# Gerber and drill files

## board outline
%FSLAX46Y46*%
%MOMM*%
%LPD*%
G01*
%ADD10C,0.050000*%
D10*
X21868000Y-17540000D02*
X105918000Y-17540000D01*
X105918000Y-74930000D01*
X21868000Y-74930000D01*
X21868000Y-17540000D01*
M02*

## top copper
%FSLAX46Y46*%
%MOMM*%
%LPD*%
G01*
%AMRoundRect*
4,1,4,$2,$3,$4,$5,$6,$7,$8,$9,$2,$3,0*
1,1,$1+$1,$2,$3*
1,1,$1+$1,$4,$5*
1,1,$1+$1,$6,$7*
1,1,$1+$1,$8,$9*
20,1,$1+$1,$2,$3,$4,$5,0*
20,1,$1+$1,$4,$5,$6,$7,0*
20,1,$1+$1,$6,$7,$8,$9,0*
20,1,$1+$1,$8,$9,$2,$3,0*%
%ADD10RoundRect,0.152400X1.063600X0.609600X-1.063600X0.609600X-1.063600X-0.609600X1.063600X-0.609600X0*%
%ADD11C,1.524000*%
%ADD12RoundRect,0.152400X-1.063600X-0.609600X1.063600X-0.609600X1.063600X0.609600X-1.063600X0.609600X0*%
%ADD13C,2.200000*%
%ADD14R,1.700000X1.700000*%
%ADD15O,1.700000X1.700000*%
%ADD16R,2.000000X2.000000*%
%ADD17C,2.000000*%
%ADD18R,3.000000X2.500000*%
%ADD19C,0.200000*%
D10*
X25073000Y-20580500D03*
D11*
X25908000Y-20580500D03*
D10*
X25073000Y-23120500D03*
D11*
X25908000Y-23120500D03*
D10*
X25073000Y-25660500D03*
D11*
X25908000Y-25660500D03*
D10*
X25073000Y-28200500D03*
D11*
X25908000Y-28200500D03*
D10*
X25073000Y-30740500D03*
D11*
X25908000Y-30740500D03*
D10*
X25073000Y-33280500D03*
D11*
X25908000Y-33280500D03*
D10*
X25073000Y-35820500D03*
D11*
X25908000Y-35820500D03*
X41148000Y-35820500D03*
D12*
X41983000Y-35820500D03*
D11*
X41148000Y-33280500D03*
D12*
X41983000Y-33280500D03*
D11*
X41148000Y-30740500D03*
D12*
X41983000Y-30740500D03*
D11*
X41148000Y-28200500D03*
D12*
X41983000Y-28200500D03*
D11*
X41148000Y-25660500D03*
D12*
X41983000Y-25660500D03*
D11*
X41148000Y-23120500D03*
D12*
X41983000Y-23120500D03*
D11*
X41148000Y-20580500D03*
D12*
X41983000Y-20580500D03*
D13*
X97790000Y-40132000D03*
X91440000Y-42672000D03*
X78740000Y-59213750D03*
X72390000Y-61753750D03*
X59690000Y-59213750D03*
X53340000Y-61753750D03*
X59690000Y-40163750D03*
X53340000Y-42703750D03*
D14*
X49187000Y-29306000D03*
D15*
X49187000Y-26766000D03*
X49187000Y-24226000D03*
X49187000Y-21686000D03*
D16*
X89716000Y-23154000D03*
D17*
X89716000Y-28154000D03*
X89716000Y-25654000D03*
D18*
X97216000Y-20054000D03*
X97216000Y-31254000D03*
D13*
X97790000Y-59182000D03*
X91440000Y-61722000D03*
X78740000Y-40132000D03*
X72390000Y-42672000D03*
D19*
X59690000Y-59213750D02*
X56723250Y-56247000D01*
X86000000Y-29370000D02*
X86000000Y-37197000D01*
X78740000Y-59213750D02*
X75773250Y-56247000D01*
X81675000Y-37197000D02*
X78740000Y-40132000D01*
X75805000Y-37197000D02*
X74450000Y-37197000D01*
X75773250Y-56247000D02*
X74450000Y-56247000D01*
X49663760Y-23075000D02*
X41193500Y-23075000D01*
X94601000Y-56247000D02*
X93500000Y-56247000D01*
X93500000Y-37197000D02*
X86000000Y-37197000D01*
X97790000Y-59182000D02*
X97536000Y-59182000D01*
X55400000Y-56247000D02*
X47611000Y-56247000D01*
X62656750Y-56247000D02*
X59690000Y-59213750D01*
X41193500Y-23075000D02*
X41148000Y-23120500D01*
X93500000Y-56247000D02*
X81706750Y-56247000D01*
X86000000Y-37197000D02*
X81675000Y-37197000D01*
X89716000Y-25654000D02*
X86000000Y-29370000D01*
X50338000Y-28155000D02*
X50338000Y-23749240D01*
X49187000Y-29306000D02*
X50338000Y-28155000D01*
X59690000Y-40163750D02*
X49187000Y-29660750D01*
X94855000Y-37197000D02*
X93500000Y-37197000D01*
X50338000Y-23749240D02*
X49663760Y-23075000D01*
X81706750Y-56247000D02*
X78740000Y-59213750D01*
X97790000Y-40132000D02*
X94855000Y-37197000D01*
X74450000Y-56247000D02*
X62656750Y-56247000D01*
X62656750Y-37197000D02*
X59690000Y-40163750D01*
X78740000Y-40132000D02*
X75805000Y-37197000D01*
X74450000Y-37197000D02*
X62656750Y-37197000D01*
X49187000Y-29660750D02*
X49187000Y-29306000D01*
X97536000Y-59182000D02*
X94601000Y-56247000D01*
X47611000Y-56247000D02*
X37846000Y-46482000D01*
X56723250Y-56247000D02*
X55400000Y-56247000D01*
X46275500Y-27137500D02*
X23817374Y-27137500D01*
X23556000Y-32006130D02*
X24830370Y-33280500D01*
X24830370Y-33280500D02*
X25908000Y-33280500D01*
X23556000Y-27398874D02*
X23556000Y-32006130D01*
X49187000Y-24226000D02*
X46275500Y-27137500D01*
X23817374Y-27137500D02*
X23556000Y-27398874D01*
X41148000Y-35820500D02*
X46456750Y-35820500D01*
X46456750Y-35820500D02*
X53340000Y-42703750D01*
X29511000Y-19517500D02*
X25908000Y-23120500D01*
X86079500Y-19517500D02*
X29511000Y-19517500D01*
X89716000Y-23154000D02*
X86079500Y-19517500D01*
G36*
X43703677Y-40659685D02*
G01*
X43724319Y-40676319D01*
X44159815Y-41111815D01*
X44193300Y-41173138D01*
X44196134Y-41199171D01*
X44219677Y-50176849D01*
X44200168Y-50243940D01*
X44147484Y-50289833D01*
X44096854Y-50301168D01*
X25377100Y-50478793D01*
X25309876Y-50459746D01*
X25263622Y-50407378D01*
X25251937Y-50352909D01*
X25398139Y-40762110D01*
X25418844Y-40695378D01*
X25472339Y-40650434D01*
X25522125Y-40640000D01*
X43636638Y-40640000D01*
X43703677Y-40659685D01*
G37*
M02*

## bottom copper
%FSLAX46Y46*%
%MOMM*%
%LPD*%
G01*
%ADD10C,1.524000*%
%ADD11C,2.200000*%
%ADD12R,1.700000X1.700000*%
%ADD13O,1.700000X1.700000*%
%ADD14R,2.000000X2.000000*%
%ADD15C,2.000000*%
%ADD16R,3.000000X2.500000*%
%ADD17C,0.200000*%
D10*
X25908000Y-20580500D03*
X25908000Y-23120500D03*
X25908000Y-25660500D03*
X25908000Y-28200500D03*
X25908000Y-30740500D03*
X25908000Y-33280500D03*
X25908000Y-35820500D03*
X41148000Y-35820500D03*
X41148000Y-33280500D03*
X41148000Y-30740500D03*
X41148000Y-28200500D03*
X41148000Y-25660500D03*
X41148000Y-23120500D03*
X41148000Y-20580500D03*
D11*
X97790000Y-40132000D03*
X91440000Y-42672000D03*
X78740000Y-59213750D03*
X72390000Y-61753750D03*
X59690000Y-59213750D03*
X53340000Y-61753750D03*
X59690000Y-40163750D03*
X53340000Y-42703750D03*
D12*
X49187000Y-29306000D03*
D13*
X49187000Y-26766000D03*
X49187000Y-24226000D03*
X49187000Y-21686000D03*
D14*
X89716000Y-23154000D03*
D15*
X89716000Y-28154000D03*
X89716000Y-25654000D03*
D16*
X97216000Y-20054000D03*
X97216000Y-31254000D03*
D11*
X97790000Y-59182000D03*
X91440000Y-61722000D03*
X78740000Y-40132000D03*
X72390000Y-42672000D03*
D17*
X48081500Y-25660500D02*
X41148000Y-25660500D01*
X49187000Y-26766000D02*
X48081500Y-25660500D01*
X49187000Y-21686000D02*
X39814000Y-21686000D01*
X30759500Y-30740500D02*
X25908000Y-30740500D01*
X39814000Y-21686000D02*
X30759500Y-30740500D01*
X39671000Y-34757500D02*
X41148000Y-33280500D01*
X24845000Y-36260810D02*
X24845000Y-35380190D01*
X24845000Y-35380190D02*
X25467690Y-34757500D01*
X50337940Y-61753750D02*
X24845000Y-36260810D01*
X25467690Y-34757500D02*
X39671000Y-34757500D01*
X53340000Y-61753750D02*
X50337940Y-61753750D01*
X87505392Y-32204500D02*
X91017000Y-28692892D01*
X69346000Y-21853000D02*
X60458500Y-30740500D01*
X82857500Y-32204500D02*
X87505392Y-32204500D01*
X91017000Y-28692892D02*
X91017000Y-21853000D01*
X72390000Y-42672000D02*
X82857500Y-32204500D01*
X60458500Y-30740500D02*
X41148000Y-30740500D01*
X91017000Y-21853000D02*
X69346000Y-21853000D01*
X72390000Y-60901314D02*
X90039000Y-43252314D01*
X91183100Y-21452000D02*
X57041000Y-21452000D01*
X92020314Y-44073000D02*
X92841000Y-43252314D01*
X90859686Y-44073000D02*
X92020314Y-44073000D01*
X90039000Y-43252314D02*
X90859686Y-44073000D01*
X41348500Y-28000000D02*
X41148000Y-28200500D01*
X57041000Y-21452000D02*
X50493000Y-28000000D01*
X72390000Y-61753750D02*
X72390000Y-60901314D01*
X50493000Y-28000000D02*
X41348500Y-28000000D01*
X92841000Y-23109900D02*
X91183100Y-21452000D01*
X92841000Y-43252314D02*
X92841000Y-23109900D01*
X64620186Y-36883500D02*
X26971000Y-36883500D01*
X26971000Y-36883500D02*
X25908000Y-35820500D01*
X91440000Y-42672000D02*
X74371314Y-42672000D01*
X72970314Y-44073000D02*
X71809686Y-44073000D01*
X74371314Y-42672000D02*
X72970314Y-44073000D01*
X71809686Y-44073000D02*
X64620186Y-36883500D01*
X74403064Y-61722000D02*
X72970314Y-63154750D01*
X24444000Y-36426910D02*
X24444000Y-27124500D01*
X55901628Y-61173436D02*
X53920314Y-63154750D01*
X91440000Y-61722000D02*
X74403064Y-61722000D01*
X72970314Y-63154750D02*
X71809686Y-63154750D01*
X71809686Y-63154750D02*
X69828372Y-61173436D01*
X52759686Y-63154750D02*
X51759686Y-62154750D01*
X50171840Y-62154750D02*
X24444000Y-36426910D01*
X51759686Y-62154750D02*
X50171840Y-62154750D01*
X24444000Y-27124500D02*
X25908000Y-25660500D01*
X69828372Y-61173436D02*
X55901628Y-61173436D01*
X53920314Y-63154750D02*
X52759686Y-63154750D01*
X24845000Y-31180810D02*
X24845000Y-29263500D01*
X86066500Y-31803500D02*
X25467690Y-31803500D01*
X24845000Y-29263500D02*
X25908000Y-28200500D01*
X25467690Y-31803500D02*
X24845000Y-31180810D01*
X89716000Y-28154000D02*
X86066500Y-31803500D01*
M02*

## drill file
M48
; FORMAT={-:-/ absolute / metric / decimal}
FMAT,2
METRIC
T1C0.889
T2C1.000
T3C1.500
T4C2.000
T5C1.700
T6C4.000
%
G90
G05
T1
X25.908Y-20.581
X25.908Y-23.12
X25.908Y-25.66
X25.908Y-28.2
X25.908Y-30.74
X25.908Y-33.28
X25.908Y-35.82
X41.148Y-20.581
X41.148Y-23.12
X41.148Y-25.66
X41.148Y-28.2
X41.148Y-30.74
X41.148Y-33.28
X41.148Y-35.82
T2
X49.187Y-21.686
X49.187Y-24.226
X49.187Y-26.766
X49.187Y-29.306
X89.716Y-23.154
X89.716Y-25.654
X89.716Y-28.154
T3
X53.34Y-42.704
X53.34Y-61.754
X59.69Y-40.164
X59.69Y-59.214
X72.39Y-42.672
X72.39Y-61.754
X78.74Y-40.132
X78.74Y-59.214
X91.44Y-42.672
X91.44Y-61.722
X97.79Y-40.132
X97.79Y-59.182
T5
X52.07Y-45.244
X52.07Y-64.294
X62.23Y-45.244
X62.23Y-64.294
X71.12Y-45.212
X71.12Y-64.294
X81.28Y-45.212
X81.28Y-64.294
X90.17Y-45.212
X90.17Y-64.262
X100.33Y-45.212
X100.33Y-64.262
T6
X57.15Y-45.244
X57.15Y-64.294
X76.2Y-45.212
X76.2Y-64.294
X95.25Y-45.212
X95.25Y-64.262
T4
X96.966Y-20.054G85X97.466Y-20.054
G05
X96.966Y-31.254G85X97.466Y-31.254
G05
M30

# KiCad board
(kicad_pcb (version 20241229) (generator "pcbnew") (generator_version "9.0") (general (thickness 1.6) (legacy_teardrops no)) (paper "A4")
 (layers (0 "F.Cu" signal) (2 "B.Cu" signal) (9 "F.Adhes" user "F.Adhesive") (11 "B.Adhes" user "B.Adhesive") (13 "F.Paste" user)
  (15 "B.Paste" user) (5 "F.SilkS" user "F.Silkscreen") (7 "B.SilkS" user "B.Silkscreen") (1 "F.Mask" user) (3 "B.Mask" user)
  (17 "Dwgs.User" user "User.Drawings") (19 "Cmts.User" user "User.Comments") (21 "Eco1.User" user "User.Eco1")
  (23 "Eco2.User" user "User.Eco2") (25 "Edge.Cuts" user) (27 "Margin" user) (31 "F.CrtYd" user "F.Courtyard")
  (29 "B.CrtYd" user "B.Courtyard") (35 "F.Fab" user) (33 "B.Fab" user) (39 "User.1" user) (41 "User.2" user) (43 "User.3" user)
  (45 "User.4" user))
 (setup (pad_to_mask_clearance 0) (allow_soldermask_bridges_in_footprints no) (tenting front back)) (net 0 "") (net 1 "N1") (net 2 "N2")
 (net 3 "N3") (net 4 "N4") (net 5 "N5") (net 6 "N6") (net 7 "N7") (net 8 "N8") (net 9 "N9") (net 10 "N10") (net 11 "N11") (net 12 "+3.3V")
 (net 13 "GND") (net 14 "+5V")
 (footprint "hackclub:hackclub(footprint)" (layer "F.Cu") (at 35 58.15)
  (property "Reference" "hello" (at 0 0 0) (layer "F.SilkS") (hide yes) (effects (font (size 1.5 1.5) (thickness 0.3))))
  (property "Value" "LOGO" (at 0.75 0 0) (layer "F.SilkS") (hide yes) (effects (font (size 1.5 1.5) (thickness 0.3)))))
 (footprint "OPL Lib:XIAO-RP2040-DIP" (layer "F.Cu") (at 33.528 28.2005)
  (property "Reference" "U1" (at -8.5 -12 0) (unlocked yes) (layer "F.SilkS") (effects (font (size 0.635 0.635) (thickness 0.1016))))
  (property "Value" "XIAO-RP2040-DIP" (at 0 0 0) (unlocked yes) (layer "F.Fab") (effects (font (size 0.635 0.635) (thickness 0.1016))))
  (pad "1" smd roundrect (at -8.455 -7.62 180) (size 2.432 1.524) (layers "F.Cu" "F.Mask") (roundrect_rratio 0.1) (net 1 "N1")
   (thermal_bridge_angle 45))
  (pad "1" thru_hole circle (at -7.62 -7.62 180) (size 1.524 1.524) (drill 0.889) (layers "*.Cu" "*.Mask") (remove_unused_layers no)
   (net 1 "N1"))
  (pad "2" smd roundrect (at -8.455 -5.08 180) (size 2.432 1.524) (layers "F.Cu" "F.Mask") (roundrect_rratio 0.1) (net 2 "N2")
   (thermal_bridge_angle 45))
  (pad "2" thru_hole circle (at -7.62 -5.08 180) (size 1.524 1.524) (drill 0.889) (layers "*.Cu" "*.Mask") (remove_unused_layers no)
   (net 2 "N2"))
  (pad "3" smd roundrect (at -8.455 -2.54 180) (size 2.432 1.524) (layers "F.Cu" "F.Mask") (roundrect_rratio 0.1) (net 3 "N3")
   (thermal_bridge_angle 45))
  (pad "3" thru_hole circle (at -7.62 -2.54 180) (size 1.524 1.524) (drill 0.889) (layers "*.Cu" "*.Mask") (remove_unused_layers no)
   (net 3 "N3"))
  (pad "4" smd roundrect (at -8.455 0 180) (size 2.432 1.524) (layers "F.Cu" "F.Mask") (roundrect_rratio 0.1) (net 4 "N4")
   (thermal_bridge_angle 45))
  (pad "4" thru_hole circle (at -7.62 0 180) (size 1.524 1.524) (drill 0.889) (layers "*.Cu" "*.Mask") (remove_unused_layers no)
   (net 4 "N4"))
  (pad "5" smd roundrect (at -8.455 2.54 180) (size 2.432 1.524) (layers "F.Cu" "F.Mask") (roundrect_rratio 0.1) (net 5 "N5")
   (thermal_bridge_angle 45))
  (pad "5" thru_hole circle (at -7.62 2.54 180) (size 1.524 1.524) (drill 0.889) (layers "*.Cu" "*.Mask") (remove_unused_layers no)
   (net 5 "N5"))
  (pad "6" smd roundrect (at -8.455 5.08 180) (size 2.432 1.524) (layers "F.Cu" "F.Mask") (roundrect_rratio 0.1) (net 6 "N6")
   (thermal_bridge_angle 45))
  (pad "6" thru_hole circle (at -7.62 5.08 180) (size 1.524 1.524) (drill 0.889) (layers "*.Cu" "*.Mask") (remove_unused_layers no)
   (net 6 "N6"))
  (pad "7" smd roundrect (at -8.455 7.62 180) (size 2.432 1.524) (layers "F.Cu" "F.Mask") (roundrect_rratio 0.1) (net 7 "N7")
   (thermal_bridge_angle 45))
  (pad "7" thru_hole circle (at -7.62 7.62 180) (size 1.524 1.524) (drill 0.889) (layers "*.Cu" "*.Mask") (remove_unused_layers no)
   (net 7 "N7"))
  (pad "8" thru_hole circle (at 7.62 7.62) (size 1.524 1.524) (drill 0.889) (layers "*.Cu" "*.Mask") (remove_unused_layers no) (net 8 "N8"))
  (pad "8" smd roundrect (at 8.455 7.62) (size 2.432 1.524) (layers "F.Cu" "F.Mask") (roundrect_rratio 0.1) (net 8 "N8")
   (thermal_bridge_angle 45))
  (pad "9" thru_hole circle (at 7.62 5.08) (size 1.524 1.524) (drill 0.889) (layers "*.Cu" "*.Mask") (remove_unused_layers no) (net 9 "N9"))
  (pad "9" smd roundrect (at 8.455 5.08) (size 2.432 1.524) (layers "F.Cu" "F.Mask") (roundrect_rratio 0.1) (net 9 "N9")
   (thermal_bridge_angle 45))
  (pad "10" thru_hole circle (at 7.62 2.54) (size 1.524 1.524) (drill 0.889) (layers "*.Cu" "*.Mask") (remove_unused_layers no)
   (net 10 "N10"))
  (pad "10" smd roundrect (at 8.455 2.54) (size 2.432 1.524) (layers "F.Cu" "F.Mask") (roundrect_rratio 0.1) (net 10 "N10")
   (thermal_bridge_angle 45))
  (pad "11" thru_hole circle (at 7.62 0) (size 1.524 1.524) (drill 0.889) (layers "*.Cu" "*.Mask") (remove_unused_layers no) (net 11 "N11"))
  (pad "11" smd roundrect (at 8.455 0) (size 2.432 1.524) (layers "F.Cu" "F.Mask") (roundrect_rratio 0.1) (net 11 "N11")
   (thermal_bridge_angle 45))
  (pad "12" thru_hole circle (at 7.62 -2.54) (size 1.524 1.524) (drill 0.889) (layers "*.Cu" "*.Mask") (remove_unused_layers no)
   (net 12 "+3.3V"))
  (pad "12" smd roundrect (at 8.455 -2.54) (size 2.432 1.524) (layers "F.Cu" "F.Mask") (roundrect_rratio 0.1) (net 12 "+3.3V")
   (thermal_bridge_angle 45))
  (pad "13" thru_hole circle (at 7.62 -5.08) (size 1.524 1.524) (drill 0.889) (layers "*.Cu" "*.Mask") (remove_unused_layers no)
   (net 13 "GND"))
  (pad "13" smd roundrect (at 8.455 -5.08) (size 2.432 1.524) (layers "F.Cu" "F.Mask") (roundrect_rratio 0.1) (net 13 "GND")
   (thermal_bridge_angle 45))
  (pad "14" thru_hole circle (at 7.62 -7.62) (size 1.524 1.524) (drill 0.889) (layers "*.Cu" "*.Mask") (remove_unused_layers no)
   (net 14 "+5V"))
  (pad "14" smd roundrect (at 8.455 -7.62) (size 2.432 1.524) (layers "F.Cu" "F.Mask") (roundrect_rratio 0.1) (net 14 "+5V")
   (thermal_bridge_angle 45)))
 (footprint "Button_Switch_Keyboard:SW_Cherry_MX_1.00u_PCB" (layer "F.Cu") (at 97.79 40.132)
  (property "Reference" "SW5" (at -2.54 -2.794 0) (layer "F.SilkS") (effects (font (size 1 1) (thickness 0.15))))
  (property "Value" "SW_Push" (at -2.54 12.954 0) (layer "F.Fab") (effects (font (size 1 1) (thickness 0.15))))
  (pad "" np_thru_hole circle (at -7.62 5.08) (size 1.7 1.7) (drill 1.7) (layers "*.Cu" "*.Mask"))
  (pad "" np_thru_hole circle (at -2.54 5.08) (size 4 4) (drill 4) (layers "*.Cu" "*.Mask"))
  (pad "" np_thru_hole circle (at 2.54 5.08) (size 1.7 1.7) (drill 1.7) (layers "*.Cu" "*.Mask"))
  (pad "1" thru_hole circle (at 0 0) (size 2.2 2.2) (drill 1.5) (layers "*.Cu" "*.Mask") (remove_unused_layers no) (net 13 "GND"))
  (pad "2" thru_hole circle (at -6.35 2.54) (size 2.2 2.2) (drill 1.5) (layers "*.Cu" "*.Mask") (remove_unused_layers no) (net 7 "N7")))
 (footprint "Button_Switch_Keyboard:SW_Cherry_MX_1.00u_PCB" (layer "F.Cu") (at 78.74 59.21375)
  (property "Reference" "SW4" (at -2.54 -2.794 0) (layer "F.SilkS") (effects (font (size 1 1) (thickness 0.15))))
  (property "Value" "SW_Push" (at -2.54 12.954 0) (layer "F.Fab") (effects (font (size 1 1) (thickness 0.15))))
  (pad "" np_thru_hole circle (at -7.62 5.08) (size 1.7 1.7) (drill 1.7) (layers "*.Cu" "*.Mask"))
  (pad "" np_thru_hole circle (at -2.54 5.08) (size 4 4) (drill 4) (layers "*.Cu" "*.Mask"))
  (pad "" np_thru_hole circle (at 2.54 5.08) (size 1.7 1.7) (drill 1.7) (layers "*.Cu" "*.Mask"))
  (pad "1" thru_hole circle (at 0 0) (size 2.2 2.2) (drill 1.5) (layers "*.Cu" "*.Mask") (remove_unused_layers no) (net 13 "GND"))
  (pad "2" thru_hole circle (at -6.35 2.54) (size 2.2 2.2) (drill 1.5) (layers "*.Cu" "*.Mask") (remove_unused_layers no) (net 11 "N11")))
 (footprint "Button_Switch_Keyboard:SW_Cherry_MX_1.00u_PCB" (layer "F.Cu") (at 59.69 59.21375)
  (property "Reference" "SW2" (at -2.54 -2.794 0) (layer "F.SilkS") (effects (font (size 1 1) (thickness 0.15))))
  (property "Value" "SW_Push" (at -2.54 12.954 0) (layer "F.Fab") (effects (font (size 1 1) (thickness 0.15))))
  (pad "" np_thru_hole circle (at -7.62 5.08) (size 1.7 1.7) (drill 1.7) (layers "*.Cu" "*.Mask"))
  (pad "" np_thru_hole circle (at -2.54 5.08) (size 4 4) (drill 4) (layers "*.Cu" "*.Mask"))
  (pad "" np_thru_hole circle (at 2.54 5.08) (size 1.7 1.7) (drill 1.7) (layers "*.Cu" "*.Mask"))
  (pad "1" thru_hole circle (at 0 0) (size 2.2 2.2) (drill 1.5) (layers "*.Cu" "*.Mask") (remove_unused_layers no) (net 13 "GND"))
  (pad "2" thru_hole circle (at -6.35 2.54) (size 2.2 2.2) (drill 1.5) (layers "*.Cu" "*.Mask") (remove_unused_layers no) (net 9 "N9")))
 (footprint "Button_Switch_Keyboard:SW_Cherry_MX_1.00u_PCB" (layer "F.Cu") (at 59.69 40.16375)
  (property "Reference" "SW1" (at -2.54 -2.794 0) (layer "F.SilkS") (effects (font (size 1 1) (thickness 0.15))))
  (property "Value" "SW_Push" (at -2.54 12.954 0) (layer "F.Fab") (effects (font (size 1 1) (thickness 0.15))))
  (pad "" np_thru_hole circle (at -7.62 5.08) (size 1.7 1.7) (drill 1.7) (layers "*.Cu" "*.Mask"))
  (pad "" np_thru_hole circle (at -2.54 5.08) (size 4 4) (drill 4) (layers "*.Cu" "*.Mask"))
  (pad "" np_thru_hole circle (at 2.54 5.08) (size 1.7 1.7) (drill 1.7) (layers "*.Cu" "*.Mask"))
  (pad "1" thru_hole circle (at 0 0) (size 2.2 2.2) (drill 1.5) (layers "*.Cu" "*.Mask") (remove_unused_layers no) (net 13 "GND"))
  (pad "2" thru_hole circle (at -6.35 2.54) (size 2.2 2.2) (drill 1.5) (layers "*.Cu" "*.Mask") (remove_unused_layers no) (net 8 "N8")))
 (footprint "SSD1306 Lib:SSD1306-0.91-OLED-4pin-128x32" (layer "F.Cu") (at 85.687 31.496 180)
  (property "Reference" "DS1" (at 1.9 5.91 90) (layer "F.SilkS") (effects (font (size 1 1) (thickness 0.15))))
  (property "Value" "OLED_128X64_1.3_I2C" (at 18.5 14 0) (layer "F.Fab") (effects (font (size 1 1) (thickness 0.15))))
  (pad "1" thru_hole rect (at 36.5 2.19 180) (size 1.7 1.7) (drill 1) (layers "*.Cu" "*.Mask") (remove_unused_layers no) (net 13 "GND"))
  (pad "2" thru_hole oval (at 36.5 4.73 180) (size 1.7 1.7) (drill 1) (layers "*.Cu" "*.Mask") (remove_unused_layers no) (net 12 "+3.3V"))
  (pad "3" thru_hole oval (at 36.5 7.27 180) (size 1.7 1.7) (drill 1) (layers "*.Cu" "*.Mask") (remove_unused_layers no) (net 6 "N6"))
  (pad "4" thru_hole oval (at 36.5 9.81 180) (size 1.7 1.7) (drill 1) (layers "*.Cu" "*.Mask") (remove_unused_layers no) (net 5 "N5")))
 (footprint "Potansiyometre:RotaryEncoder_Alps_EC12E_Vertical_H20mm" (layer "F.Cu") (at 89.716 23.154)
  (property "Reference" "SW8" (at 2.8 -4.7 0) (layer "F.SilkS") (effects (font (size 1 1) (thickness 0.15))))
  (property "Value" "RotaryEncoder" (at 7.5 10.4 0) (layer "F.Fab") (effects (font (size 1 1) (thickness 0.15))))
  (pad "A" thru_hole rect (at 0 0) (size 2 2) (drill 1) (layers "*.Cu" "*.Mask") (remove_unused_layers no) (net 2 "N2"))
  (pad "B" thru_hole circle (at 0 5) (size 2 2) (drill 1) (layers "*.Cu" "*.Mask") (remove_unused_layers no) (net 4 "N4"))
  (pad "C" thru_hole circle (at 0 2.5) (size 2 2) (drill 1) (layers "*.Cu" "*.Mask") (remove_unused_layers no) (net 13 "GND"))
  (pad "MP" thru_hole rect (at 7.5 -3.1) (size 3 2.5) (drill oval 2.5 2) (layers "*.Cu" "*.Mask") (remove_unused_layers no))
  (pad "MP" thru_hole rect (at 7.5 8.1) (size 3 2.5) (drill oval 2.5 2) (layers "*.Cu" "*.Mask") (remove_unused_layers no)))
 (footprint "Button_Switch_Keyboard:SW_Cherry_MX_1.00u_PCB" (layer "F.Cu") (at 97.79 59.182)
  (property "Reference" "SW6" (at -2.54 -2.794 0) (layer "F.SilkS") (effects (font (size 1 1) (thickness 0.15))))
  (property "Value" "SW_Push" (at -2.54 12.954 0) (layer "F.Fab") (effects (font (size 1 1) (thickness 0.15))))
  (pad "" np_thru_hole circle (at -7.62 5.08) (size 1.7 1.7) (drill 1.7) (layers "*.Cu" "*.Mask"))
  (pad "" np_thru_hole circle (at -2.54 5.08) (size 4 4) (drill 4) (layers "*.Cu" "*.Mask"))
  (pad "" np_thru_hole circle (at 2.54 5.08) (size 1.7 1.7) (drill 1.7) (layers "*.Cu" "*.Mask"))
  (pad "1" thru_hole circle (at 0 0) (size 2.2 2.2) (drill 1.5) (layers "*.Cu" "*.Mask") (remove_unused_layers no) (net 13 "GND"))
  (pad "2" thru_hole circle (at -6.35 2.54) (size 2.2 2.2) (drill 1.5) (layers "*.Cu" "*.Mask") (remove_unused_layers no) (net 3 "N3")))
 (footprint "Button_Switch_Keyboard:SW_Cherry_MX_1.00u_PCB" (layer "F.Cu") (at 78.74 40.132)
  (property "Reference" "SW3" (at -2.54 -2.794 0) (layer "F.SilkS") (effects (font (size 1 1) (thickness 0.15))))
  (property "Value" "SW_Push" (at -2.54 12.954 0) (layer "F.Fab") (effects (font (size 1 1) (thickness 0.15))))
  (pad "" np_thru_hole circle (at -7.62 5.08) (size 1.7 1.7) (drill 1.7) (layers "*.Cu" "*.Mask"))
  (pad "" np_thru_hole circle (at -2.54 5.08) (size 4 4) (drill 4) (layers "*.Cu" "*.Mask"))
  (pad "" np_thru_hole circle (at 2.54 5.08) (size 1.7 1.7) (drill 1.7) (layers "*.Cu" "*.Mask"))
  (pad "1" thru_hole circle (at 0 0) (size 2.2 2.2) (drill 1.5) (layers "*.Cu" "*.Mask") (remove_unused_layers no) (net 13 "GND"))
  (pad "2" thru_hole circle (at -6.35 2.54) (size 2.2 2.2) (drill 1.5) (layers "*.Cu" "*.Mask") (remove_unused_layers no) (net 10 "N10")))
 (gr_rect (start 21.868 17.54) (end 105.918 74.93) (stroke (width 0.05) (type default)) (fill no) (layer "Edge.Cuts"))
 (segment (start 59.69 59.21375) (end 56.72325 56.247) (width 0.2) (layer "F.Cu") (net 13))
 (segment (start 86 29.37) (end 86 37.197) (width 0.2) (layer "F.Cu") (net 13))
 (segment (start 78.74 59.21375) (end 75.77325 56.247) (width 0.2) (layer "F.Cu") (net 13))
 (segment (start 81.675 37.197) (end 78.74 40.132) (width 0.2) (layer "F.Cu") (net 13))
 (segment (start 75.805 37.197) (end 74.45 37.197) (width 0.2) (layer "F.Cu") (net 13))
 (segment (start 75.77325 56.247) (end 74.45 56.247) (width 0.2) (layer "F.Cu") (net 13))
 (segment (start 49.66376 23.075) (end 41.1935 23.075) (width 0.2) (layer "F.Cu") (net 13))
 (segment (start 94.601 56.247) (end 93.5 56.247) (width 0.2) (layer "F.Cu") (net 13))
 (segment (start 93.5 37.197) (end 86 37.197) (width 0.2) (layer "F.Cu") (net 13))
 (segment (start 97.79 59.182) (end 97.536 59.182) (width 0.2) (layer "F.Cu") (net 13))
 (segment (start 55.4 56.247) (end 47.611 56.247) (width 0.2) (layer "F.Cu") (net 13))
 (segment (start 62.65675 56.247) (end 59.69 59.21375) (width 0.2) (layer "F.Cu") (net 13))
 (segment (start 41.1935 23.075) (end 41.148 23.1205) (width 0.2) (layer "F.Cu") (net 13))
 (segment (start 93.5 56.247) (end 81.70675 56.247) (width 0.2) (layer "F.Cu") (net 13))
 (segment (start 86 37.197) (end 81.675 37.197) (width 0.2) (layer "F.Cu") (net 13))
 (segment (start 89.716 25.654) (end 86 29.37) (width 0.2) (layer "F.Cu") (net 13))
 (segment (start 50.338 28.155) (end 50.338 23.74924) (width 0.2) (layer "F.Cu") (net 13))
 (segment (start 49.187 29.306) (end 50.338 28.155) (width 0.2) (layer "F.Cu") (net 13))
 (segment (start 59.69 40.16375) (end 49.187 29.66075) (width 0.2) (layer "F.Cu") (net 13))
 (segment (start 94.855 37.197) (end 93.5 37.197) (width 0.2) (layer "F.Cu") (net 13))
 (segment (start 50.338 23.74924) (end 49.66376 23.075) (width 0.2) (layer "F.Cu") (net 13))
 (segment (start 81.70675 56.247) (end 78.74 59.21375) (width 0.2) (layer "F.Cu") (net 13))
 (segment (start 97.79 40.132) (end 94.855 37.197) (width 0.2) (layer "F.Cu") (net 13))
 (segment (start 74.45 56.247) (end 62.65675 56.247) (width 0.2) (layer "F.Cu") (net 13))
 (segment (start 62.65675 37.197) (end 59.69 40.16375) (width 0.2) (layer "F.Cu") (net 13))
 (segment (start 78.74 40.132) (end 75.805 37.197) (width 0.2) (layer "F.Cu") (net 13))
 (segment (start 74.45 37.197) (end 62.65675 37.197) (width 0.2) (layer "F.Cu") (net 13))
 (segment (start 49.187 29.66075) (end 49.187 29.306) (width 0.2) (layer "F.Cu") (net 13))
 (segment (start 97.536 59.182) (end 94.601 56.247) (width 0.2) (layer "F.Cu") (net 13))
 (segment (start 47.611 56.247) (end 37.846 46.482) (width 0.2) (layer "F.Cu") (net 13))
 (segment (start 56.72325 56.247) (end 55.4 56.247) (width 0.2) (layer "F.Cu") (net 13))
 (segment (start 48.0815 25.6605) (end 41.148 25.6605) (width 0.2) (layer "B.Cu") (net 12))
 (segment (start 49.187 26.766) (end 48.0815 25.6605) (width 0.2) (layer "B.Cu") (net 12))
 (segment (start 49.187 21.686) (end 39.814 21.686) (width 0.2) (layer "B.Cu") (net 5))
 (segment (start 30.7595 30.7405) (end 25.908 30.7405) (width 0.2) (layer "B.Cu") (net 5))
 (segment (start 39.814 21.686) (end 30.7595 30.7405) (width 0.2) (layer "B.Cu") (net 5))
 (segment (start 46.2755 27.1375) (end 23.817374 27.1375) (width 0.2) (layer "F.Cu") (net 6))
 (segment (start 23.556 32.00613) (end 24.83037 33.2805) (width 0.2) (layer "F.Cu") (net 6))
 (segment (start 24.83037 33.2805) (end 25.908 33.2805) (width 0.2) (layer "F.Cu") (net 6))
 (segment (start 23.556 27.398874) (end 23.556 32.00613) (width 0.2) (layer "F.Cu") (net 6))
 (segment (start 49.187 24.226) (end 46.2755 27.1375) (width 0.2) (layer "F.Cu") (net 6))
 (segment (start 23.817374 27.1375) (end 23.556 27.398874) (width 0.2) (layer "F.Cu") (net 6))
 (segment (start 41.148 35.8205) (end 46.45675 35.8205) (width 0.2) (layer "F.Cu") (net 8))
 (segment (start 46.45675 35.8205) (end 53.34 42.70375) (width 0.2) (layer "F.Cu") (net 8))
 (segment (start 39.671 34.7575) (end 41.148 33.2805) (width 0.2) (layer "B.Cu") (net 9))
 (segment (start 24.845 36.26081) (end 24.845 35.38019) (width 0.2) (layer "B.Cu") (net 9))
 (segment (start 24.845 35.38019) (end 25.46769 34.7575) (width 0.2) (layer "B.Cu") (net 9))
 (segment (start 50.33794 61.75375) (end 24.845 36.26081) (width 0.2) (layer "B.Cu") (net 9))
 (segment (start 25.46769 34.7575) (end 39.671 34.7575) (width 0.2) (layer "B.Cu") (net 9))
 (segment (start 53.34 61.75375) (end 50.33794 61.75375) (width 0.2) (layer "B.Cu") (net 9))
 (segment (start 87.505392 32.2045) (end 91.017 28.692892) (width 0.2) (layer "B.Cu") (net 10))
 (segment (start 69.346 21.853) (end 60.4585 30.7405) (width 0.2) (layer "B.Cu") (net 10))
 (segment (start 82.8575 32.2045) (end 87.505392 32.2045) (width 0.2) (layer "B.Cu") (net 10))
 (segment (start 91.017 28.692892) (end 91.017 21.853) (width 0.2) (layer "B.Cu") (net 10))
 (segment (start 72.39 42.672) (end 82.8575 32.2045) (width 0.2) (layer "B.Cu") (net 10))
 (segment (start 60.4585 30.7405) (end 41.148 30.7405) (width 0.2) (layer "B.Cu") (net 10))
 (segment (start 91.017 21.853) (end 69.346 21.853) (width 0.2) (layer "B.Cu") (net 10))
 (segment (start 72.39 60.901314) (end 90.039 43.252314) (width 0.2) (layer "B.Cu") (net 11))
 (segment (start 91.1831 21.452) (end 57.041 21.452) (width 0.2) (layer "B.Cu") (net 11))
 (segment (start 92.020314 44.073) (end 92.841 43.252314) (width 0.2) (layer "B.Cu") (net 11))
 (segment (start 90.859686 44.073) (end 92.020314 44.073) (width 0.2) (layer "B.Cu") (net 11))
 (segment (start 90.039 43.252314) (end 90.859686 44.073) (width 0.2) (layer "B.Cu") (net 11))
 (segment (start 41.3485 28) (end 41.148 28.2005) (width 0.2) (layer "B.Cu") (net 11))
 (segment (start 57.041 21.452) (end 50.493 28) (width 0.2) (layer "B.Cu") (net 11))
 (segment (start 72.39 61.75375) (end 72.39 60.901314) (width 0.2) (layer "B.Cu") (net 11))
 (segment (start 50.493 28) (end 41.3485 28) (width 0.2) (layer "B.Cu") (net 11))
 (segment (start 92.841 23.1099) (end 91.1831 21.452) (width 0.2) (layer "B.Cu") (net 11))
 (segment (start 92.841 43.252314) (end 92.841 23.1099) (width 0.2) (layer "B.Cu") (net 11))
 (segment (start 64.620186 36.8835) (end 26.971 36.8835) (width 0.2) (layer "B.Cu") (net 7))
 (segment (start 26.971 36.8835) (end 25.908 35.8205) (width 0.2) (layer "B.Cu") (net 7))
 (segment (start 91.44 42.672) (end 74.371314 42.672) (width 0.2) (layer "B.Cu") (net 7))
 (segment (start 72.970314 44.073) (end 71.809686 44.073) (width 0.2) (layer "B.Cu") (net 7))
 (segment (start 74.371314 42.672) (end 72.970314 44.073) (width 0.2) (layer "B.Cu") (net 7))
 (segment (start 71.809686 44.073) (end 64.620186 36.8835) (width 0.2) (layer "B.Cu") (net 7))
 (segment (start 74.403064 61.722) (end 72.970314 63.15475) (width 0.2) (layer "B.Cu") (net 3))
 (segment (start 24.444 36.42691) (end 24.444 27.1245) (width 0.2) (layer "B.Cu") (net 3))
 (segment (start 55.901628 61.173436) (end 53.920314 63.15475) (width 0.2) (layer "B.Cu") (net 3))
 (segment (start 91.44 61.722) (end 74.403064 61.722) (width 0.2) (layer "B.Cu") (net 3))
 (segment (start 72.970314 63.15475) (end 71.809686 63.15475) (width 0.2) (layer "B.Cu") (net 3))
 (segment (start 71.809686 63.15475) (end 69.828372 61.173436) (width 0.2) (layer "B.Cu") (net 3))
 (segment (start 52.759686 63.15475) (end 51.759686 62.15475) (width 0.2) (layer "B.Cu") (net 3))
 (segment (start 50.17184 62.15475) (end 24.444 36.42691) (width 0.2) (layer "B.Cu") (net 3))
 (segment (start 51.759686 62.15475) (end 50.17184 62.15475) (width 0.2) (layer "B.Cu") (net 3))
 (segment (start 24.444 27.1245) (end 25.908 25.6605) (width 0.2) (layer "B.Cu") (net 3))
 (segment (start 69.828372 61.173436) (end 55.901628 61.173436) (width 0.2) (layer "B.Cu") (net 3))
 (segment (start 53.920314 63.15475) (end 52.759686 63.15475) (width 0.2) (layer "B.Cu") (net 3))
 (segment (start 24.845 31.18081) (end 24.845 29.2635) (width 0.2) (layer "B.Cu") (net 4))
 (segment (start 86.0665 31.8035) (end 25.46769 31.8035) (width 0.2) (layer "B.Cu") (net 4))
 (segment (start 24.845 29.2635) (end 25.908 28.2005) (width 0.2) (layer "B.Cu") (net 4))
 (segment (start 25.46769 31.8035) (end 24.845 31.18081) (width 0.2) (layer "B.Cu") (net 4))
 (segment (start 89.716 28.154) (end 86.0665 31.8035) (width 0.2) (layer "B.Cu") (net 4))
 (segment (start 29.511 19.5175) (end 25.908 23.1205) (width 0.2) (layer "F.Cu") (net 2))
 (segment (start 86.0795 19.5175) (end 29.511 19.5175) (width 0.2) (layer "F.Cu") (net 2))
 (segment (start 89.716 23.154) (end 86.0795 19.5175) (width 0.2) (layer "F.Cu") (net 2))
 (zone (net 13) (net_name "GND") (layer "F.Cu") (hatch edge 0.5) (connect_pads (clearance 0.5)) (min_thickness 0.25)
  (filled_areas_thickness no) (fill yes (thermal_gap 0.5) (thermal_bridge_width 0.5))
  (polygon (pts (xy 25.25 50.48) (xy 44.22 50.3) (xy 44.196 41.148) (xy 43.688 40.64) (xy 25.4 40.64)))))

